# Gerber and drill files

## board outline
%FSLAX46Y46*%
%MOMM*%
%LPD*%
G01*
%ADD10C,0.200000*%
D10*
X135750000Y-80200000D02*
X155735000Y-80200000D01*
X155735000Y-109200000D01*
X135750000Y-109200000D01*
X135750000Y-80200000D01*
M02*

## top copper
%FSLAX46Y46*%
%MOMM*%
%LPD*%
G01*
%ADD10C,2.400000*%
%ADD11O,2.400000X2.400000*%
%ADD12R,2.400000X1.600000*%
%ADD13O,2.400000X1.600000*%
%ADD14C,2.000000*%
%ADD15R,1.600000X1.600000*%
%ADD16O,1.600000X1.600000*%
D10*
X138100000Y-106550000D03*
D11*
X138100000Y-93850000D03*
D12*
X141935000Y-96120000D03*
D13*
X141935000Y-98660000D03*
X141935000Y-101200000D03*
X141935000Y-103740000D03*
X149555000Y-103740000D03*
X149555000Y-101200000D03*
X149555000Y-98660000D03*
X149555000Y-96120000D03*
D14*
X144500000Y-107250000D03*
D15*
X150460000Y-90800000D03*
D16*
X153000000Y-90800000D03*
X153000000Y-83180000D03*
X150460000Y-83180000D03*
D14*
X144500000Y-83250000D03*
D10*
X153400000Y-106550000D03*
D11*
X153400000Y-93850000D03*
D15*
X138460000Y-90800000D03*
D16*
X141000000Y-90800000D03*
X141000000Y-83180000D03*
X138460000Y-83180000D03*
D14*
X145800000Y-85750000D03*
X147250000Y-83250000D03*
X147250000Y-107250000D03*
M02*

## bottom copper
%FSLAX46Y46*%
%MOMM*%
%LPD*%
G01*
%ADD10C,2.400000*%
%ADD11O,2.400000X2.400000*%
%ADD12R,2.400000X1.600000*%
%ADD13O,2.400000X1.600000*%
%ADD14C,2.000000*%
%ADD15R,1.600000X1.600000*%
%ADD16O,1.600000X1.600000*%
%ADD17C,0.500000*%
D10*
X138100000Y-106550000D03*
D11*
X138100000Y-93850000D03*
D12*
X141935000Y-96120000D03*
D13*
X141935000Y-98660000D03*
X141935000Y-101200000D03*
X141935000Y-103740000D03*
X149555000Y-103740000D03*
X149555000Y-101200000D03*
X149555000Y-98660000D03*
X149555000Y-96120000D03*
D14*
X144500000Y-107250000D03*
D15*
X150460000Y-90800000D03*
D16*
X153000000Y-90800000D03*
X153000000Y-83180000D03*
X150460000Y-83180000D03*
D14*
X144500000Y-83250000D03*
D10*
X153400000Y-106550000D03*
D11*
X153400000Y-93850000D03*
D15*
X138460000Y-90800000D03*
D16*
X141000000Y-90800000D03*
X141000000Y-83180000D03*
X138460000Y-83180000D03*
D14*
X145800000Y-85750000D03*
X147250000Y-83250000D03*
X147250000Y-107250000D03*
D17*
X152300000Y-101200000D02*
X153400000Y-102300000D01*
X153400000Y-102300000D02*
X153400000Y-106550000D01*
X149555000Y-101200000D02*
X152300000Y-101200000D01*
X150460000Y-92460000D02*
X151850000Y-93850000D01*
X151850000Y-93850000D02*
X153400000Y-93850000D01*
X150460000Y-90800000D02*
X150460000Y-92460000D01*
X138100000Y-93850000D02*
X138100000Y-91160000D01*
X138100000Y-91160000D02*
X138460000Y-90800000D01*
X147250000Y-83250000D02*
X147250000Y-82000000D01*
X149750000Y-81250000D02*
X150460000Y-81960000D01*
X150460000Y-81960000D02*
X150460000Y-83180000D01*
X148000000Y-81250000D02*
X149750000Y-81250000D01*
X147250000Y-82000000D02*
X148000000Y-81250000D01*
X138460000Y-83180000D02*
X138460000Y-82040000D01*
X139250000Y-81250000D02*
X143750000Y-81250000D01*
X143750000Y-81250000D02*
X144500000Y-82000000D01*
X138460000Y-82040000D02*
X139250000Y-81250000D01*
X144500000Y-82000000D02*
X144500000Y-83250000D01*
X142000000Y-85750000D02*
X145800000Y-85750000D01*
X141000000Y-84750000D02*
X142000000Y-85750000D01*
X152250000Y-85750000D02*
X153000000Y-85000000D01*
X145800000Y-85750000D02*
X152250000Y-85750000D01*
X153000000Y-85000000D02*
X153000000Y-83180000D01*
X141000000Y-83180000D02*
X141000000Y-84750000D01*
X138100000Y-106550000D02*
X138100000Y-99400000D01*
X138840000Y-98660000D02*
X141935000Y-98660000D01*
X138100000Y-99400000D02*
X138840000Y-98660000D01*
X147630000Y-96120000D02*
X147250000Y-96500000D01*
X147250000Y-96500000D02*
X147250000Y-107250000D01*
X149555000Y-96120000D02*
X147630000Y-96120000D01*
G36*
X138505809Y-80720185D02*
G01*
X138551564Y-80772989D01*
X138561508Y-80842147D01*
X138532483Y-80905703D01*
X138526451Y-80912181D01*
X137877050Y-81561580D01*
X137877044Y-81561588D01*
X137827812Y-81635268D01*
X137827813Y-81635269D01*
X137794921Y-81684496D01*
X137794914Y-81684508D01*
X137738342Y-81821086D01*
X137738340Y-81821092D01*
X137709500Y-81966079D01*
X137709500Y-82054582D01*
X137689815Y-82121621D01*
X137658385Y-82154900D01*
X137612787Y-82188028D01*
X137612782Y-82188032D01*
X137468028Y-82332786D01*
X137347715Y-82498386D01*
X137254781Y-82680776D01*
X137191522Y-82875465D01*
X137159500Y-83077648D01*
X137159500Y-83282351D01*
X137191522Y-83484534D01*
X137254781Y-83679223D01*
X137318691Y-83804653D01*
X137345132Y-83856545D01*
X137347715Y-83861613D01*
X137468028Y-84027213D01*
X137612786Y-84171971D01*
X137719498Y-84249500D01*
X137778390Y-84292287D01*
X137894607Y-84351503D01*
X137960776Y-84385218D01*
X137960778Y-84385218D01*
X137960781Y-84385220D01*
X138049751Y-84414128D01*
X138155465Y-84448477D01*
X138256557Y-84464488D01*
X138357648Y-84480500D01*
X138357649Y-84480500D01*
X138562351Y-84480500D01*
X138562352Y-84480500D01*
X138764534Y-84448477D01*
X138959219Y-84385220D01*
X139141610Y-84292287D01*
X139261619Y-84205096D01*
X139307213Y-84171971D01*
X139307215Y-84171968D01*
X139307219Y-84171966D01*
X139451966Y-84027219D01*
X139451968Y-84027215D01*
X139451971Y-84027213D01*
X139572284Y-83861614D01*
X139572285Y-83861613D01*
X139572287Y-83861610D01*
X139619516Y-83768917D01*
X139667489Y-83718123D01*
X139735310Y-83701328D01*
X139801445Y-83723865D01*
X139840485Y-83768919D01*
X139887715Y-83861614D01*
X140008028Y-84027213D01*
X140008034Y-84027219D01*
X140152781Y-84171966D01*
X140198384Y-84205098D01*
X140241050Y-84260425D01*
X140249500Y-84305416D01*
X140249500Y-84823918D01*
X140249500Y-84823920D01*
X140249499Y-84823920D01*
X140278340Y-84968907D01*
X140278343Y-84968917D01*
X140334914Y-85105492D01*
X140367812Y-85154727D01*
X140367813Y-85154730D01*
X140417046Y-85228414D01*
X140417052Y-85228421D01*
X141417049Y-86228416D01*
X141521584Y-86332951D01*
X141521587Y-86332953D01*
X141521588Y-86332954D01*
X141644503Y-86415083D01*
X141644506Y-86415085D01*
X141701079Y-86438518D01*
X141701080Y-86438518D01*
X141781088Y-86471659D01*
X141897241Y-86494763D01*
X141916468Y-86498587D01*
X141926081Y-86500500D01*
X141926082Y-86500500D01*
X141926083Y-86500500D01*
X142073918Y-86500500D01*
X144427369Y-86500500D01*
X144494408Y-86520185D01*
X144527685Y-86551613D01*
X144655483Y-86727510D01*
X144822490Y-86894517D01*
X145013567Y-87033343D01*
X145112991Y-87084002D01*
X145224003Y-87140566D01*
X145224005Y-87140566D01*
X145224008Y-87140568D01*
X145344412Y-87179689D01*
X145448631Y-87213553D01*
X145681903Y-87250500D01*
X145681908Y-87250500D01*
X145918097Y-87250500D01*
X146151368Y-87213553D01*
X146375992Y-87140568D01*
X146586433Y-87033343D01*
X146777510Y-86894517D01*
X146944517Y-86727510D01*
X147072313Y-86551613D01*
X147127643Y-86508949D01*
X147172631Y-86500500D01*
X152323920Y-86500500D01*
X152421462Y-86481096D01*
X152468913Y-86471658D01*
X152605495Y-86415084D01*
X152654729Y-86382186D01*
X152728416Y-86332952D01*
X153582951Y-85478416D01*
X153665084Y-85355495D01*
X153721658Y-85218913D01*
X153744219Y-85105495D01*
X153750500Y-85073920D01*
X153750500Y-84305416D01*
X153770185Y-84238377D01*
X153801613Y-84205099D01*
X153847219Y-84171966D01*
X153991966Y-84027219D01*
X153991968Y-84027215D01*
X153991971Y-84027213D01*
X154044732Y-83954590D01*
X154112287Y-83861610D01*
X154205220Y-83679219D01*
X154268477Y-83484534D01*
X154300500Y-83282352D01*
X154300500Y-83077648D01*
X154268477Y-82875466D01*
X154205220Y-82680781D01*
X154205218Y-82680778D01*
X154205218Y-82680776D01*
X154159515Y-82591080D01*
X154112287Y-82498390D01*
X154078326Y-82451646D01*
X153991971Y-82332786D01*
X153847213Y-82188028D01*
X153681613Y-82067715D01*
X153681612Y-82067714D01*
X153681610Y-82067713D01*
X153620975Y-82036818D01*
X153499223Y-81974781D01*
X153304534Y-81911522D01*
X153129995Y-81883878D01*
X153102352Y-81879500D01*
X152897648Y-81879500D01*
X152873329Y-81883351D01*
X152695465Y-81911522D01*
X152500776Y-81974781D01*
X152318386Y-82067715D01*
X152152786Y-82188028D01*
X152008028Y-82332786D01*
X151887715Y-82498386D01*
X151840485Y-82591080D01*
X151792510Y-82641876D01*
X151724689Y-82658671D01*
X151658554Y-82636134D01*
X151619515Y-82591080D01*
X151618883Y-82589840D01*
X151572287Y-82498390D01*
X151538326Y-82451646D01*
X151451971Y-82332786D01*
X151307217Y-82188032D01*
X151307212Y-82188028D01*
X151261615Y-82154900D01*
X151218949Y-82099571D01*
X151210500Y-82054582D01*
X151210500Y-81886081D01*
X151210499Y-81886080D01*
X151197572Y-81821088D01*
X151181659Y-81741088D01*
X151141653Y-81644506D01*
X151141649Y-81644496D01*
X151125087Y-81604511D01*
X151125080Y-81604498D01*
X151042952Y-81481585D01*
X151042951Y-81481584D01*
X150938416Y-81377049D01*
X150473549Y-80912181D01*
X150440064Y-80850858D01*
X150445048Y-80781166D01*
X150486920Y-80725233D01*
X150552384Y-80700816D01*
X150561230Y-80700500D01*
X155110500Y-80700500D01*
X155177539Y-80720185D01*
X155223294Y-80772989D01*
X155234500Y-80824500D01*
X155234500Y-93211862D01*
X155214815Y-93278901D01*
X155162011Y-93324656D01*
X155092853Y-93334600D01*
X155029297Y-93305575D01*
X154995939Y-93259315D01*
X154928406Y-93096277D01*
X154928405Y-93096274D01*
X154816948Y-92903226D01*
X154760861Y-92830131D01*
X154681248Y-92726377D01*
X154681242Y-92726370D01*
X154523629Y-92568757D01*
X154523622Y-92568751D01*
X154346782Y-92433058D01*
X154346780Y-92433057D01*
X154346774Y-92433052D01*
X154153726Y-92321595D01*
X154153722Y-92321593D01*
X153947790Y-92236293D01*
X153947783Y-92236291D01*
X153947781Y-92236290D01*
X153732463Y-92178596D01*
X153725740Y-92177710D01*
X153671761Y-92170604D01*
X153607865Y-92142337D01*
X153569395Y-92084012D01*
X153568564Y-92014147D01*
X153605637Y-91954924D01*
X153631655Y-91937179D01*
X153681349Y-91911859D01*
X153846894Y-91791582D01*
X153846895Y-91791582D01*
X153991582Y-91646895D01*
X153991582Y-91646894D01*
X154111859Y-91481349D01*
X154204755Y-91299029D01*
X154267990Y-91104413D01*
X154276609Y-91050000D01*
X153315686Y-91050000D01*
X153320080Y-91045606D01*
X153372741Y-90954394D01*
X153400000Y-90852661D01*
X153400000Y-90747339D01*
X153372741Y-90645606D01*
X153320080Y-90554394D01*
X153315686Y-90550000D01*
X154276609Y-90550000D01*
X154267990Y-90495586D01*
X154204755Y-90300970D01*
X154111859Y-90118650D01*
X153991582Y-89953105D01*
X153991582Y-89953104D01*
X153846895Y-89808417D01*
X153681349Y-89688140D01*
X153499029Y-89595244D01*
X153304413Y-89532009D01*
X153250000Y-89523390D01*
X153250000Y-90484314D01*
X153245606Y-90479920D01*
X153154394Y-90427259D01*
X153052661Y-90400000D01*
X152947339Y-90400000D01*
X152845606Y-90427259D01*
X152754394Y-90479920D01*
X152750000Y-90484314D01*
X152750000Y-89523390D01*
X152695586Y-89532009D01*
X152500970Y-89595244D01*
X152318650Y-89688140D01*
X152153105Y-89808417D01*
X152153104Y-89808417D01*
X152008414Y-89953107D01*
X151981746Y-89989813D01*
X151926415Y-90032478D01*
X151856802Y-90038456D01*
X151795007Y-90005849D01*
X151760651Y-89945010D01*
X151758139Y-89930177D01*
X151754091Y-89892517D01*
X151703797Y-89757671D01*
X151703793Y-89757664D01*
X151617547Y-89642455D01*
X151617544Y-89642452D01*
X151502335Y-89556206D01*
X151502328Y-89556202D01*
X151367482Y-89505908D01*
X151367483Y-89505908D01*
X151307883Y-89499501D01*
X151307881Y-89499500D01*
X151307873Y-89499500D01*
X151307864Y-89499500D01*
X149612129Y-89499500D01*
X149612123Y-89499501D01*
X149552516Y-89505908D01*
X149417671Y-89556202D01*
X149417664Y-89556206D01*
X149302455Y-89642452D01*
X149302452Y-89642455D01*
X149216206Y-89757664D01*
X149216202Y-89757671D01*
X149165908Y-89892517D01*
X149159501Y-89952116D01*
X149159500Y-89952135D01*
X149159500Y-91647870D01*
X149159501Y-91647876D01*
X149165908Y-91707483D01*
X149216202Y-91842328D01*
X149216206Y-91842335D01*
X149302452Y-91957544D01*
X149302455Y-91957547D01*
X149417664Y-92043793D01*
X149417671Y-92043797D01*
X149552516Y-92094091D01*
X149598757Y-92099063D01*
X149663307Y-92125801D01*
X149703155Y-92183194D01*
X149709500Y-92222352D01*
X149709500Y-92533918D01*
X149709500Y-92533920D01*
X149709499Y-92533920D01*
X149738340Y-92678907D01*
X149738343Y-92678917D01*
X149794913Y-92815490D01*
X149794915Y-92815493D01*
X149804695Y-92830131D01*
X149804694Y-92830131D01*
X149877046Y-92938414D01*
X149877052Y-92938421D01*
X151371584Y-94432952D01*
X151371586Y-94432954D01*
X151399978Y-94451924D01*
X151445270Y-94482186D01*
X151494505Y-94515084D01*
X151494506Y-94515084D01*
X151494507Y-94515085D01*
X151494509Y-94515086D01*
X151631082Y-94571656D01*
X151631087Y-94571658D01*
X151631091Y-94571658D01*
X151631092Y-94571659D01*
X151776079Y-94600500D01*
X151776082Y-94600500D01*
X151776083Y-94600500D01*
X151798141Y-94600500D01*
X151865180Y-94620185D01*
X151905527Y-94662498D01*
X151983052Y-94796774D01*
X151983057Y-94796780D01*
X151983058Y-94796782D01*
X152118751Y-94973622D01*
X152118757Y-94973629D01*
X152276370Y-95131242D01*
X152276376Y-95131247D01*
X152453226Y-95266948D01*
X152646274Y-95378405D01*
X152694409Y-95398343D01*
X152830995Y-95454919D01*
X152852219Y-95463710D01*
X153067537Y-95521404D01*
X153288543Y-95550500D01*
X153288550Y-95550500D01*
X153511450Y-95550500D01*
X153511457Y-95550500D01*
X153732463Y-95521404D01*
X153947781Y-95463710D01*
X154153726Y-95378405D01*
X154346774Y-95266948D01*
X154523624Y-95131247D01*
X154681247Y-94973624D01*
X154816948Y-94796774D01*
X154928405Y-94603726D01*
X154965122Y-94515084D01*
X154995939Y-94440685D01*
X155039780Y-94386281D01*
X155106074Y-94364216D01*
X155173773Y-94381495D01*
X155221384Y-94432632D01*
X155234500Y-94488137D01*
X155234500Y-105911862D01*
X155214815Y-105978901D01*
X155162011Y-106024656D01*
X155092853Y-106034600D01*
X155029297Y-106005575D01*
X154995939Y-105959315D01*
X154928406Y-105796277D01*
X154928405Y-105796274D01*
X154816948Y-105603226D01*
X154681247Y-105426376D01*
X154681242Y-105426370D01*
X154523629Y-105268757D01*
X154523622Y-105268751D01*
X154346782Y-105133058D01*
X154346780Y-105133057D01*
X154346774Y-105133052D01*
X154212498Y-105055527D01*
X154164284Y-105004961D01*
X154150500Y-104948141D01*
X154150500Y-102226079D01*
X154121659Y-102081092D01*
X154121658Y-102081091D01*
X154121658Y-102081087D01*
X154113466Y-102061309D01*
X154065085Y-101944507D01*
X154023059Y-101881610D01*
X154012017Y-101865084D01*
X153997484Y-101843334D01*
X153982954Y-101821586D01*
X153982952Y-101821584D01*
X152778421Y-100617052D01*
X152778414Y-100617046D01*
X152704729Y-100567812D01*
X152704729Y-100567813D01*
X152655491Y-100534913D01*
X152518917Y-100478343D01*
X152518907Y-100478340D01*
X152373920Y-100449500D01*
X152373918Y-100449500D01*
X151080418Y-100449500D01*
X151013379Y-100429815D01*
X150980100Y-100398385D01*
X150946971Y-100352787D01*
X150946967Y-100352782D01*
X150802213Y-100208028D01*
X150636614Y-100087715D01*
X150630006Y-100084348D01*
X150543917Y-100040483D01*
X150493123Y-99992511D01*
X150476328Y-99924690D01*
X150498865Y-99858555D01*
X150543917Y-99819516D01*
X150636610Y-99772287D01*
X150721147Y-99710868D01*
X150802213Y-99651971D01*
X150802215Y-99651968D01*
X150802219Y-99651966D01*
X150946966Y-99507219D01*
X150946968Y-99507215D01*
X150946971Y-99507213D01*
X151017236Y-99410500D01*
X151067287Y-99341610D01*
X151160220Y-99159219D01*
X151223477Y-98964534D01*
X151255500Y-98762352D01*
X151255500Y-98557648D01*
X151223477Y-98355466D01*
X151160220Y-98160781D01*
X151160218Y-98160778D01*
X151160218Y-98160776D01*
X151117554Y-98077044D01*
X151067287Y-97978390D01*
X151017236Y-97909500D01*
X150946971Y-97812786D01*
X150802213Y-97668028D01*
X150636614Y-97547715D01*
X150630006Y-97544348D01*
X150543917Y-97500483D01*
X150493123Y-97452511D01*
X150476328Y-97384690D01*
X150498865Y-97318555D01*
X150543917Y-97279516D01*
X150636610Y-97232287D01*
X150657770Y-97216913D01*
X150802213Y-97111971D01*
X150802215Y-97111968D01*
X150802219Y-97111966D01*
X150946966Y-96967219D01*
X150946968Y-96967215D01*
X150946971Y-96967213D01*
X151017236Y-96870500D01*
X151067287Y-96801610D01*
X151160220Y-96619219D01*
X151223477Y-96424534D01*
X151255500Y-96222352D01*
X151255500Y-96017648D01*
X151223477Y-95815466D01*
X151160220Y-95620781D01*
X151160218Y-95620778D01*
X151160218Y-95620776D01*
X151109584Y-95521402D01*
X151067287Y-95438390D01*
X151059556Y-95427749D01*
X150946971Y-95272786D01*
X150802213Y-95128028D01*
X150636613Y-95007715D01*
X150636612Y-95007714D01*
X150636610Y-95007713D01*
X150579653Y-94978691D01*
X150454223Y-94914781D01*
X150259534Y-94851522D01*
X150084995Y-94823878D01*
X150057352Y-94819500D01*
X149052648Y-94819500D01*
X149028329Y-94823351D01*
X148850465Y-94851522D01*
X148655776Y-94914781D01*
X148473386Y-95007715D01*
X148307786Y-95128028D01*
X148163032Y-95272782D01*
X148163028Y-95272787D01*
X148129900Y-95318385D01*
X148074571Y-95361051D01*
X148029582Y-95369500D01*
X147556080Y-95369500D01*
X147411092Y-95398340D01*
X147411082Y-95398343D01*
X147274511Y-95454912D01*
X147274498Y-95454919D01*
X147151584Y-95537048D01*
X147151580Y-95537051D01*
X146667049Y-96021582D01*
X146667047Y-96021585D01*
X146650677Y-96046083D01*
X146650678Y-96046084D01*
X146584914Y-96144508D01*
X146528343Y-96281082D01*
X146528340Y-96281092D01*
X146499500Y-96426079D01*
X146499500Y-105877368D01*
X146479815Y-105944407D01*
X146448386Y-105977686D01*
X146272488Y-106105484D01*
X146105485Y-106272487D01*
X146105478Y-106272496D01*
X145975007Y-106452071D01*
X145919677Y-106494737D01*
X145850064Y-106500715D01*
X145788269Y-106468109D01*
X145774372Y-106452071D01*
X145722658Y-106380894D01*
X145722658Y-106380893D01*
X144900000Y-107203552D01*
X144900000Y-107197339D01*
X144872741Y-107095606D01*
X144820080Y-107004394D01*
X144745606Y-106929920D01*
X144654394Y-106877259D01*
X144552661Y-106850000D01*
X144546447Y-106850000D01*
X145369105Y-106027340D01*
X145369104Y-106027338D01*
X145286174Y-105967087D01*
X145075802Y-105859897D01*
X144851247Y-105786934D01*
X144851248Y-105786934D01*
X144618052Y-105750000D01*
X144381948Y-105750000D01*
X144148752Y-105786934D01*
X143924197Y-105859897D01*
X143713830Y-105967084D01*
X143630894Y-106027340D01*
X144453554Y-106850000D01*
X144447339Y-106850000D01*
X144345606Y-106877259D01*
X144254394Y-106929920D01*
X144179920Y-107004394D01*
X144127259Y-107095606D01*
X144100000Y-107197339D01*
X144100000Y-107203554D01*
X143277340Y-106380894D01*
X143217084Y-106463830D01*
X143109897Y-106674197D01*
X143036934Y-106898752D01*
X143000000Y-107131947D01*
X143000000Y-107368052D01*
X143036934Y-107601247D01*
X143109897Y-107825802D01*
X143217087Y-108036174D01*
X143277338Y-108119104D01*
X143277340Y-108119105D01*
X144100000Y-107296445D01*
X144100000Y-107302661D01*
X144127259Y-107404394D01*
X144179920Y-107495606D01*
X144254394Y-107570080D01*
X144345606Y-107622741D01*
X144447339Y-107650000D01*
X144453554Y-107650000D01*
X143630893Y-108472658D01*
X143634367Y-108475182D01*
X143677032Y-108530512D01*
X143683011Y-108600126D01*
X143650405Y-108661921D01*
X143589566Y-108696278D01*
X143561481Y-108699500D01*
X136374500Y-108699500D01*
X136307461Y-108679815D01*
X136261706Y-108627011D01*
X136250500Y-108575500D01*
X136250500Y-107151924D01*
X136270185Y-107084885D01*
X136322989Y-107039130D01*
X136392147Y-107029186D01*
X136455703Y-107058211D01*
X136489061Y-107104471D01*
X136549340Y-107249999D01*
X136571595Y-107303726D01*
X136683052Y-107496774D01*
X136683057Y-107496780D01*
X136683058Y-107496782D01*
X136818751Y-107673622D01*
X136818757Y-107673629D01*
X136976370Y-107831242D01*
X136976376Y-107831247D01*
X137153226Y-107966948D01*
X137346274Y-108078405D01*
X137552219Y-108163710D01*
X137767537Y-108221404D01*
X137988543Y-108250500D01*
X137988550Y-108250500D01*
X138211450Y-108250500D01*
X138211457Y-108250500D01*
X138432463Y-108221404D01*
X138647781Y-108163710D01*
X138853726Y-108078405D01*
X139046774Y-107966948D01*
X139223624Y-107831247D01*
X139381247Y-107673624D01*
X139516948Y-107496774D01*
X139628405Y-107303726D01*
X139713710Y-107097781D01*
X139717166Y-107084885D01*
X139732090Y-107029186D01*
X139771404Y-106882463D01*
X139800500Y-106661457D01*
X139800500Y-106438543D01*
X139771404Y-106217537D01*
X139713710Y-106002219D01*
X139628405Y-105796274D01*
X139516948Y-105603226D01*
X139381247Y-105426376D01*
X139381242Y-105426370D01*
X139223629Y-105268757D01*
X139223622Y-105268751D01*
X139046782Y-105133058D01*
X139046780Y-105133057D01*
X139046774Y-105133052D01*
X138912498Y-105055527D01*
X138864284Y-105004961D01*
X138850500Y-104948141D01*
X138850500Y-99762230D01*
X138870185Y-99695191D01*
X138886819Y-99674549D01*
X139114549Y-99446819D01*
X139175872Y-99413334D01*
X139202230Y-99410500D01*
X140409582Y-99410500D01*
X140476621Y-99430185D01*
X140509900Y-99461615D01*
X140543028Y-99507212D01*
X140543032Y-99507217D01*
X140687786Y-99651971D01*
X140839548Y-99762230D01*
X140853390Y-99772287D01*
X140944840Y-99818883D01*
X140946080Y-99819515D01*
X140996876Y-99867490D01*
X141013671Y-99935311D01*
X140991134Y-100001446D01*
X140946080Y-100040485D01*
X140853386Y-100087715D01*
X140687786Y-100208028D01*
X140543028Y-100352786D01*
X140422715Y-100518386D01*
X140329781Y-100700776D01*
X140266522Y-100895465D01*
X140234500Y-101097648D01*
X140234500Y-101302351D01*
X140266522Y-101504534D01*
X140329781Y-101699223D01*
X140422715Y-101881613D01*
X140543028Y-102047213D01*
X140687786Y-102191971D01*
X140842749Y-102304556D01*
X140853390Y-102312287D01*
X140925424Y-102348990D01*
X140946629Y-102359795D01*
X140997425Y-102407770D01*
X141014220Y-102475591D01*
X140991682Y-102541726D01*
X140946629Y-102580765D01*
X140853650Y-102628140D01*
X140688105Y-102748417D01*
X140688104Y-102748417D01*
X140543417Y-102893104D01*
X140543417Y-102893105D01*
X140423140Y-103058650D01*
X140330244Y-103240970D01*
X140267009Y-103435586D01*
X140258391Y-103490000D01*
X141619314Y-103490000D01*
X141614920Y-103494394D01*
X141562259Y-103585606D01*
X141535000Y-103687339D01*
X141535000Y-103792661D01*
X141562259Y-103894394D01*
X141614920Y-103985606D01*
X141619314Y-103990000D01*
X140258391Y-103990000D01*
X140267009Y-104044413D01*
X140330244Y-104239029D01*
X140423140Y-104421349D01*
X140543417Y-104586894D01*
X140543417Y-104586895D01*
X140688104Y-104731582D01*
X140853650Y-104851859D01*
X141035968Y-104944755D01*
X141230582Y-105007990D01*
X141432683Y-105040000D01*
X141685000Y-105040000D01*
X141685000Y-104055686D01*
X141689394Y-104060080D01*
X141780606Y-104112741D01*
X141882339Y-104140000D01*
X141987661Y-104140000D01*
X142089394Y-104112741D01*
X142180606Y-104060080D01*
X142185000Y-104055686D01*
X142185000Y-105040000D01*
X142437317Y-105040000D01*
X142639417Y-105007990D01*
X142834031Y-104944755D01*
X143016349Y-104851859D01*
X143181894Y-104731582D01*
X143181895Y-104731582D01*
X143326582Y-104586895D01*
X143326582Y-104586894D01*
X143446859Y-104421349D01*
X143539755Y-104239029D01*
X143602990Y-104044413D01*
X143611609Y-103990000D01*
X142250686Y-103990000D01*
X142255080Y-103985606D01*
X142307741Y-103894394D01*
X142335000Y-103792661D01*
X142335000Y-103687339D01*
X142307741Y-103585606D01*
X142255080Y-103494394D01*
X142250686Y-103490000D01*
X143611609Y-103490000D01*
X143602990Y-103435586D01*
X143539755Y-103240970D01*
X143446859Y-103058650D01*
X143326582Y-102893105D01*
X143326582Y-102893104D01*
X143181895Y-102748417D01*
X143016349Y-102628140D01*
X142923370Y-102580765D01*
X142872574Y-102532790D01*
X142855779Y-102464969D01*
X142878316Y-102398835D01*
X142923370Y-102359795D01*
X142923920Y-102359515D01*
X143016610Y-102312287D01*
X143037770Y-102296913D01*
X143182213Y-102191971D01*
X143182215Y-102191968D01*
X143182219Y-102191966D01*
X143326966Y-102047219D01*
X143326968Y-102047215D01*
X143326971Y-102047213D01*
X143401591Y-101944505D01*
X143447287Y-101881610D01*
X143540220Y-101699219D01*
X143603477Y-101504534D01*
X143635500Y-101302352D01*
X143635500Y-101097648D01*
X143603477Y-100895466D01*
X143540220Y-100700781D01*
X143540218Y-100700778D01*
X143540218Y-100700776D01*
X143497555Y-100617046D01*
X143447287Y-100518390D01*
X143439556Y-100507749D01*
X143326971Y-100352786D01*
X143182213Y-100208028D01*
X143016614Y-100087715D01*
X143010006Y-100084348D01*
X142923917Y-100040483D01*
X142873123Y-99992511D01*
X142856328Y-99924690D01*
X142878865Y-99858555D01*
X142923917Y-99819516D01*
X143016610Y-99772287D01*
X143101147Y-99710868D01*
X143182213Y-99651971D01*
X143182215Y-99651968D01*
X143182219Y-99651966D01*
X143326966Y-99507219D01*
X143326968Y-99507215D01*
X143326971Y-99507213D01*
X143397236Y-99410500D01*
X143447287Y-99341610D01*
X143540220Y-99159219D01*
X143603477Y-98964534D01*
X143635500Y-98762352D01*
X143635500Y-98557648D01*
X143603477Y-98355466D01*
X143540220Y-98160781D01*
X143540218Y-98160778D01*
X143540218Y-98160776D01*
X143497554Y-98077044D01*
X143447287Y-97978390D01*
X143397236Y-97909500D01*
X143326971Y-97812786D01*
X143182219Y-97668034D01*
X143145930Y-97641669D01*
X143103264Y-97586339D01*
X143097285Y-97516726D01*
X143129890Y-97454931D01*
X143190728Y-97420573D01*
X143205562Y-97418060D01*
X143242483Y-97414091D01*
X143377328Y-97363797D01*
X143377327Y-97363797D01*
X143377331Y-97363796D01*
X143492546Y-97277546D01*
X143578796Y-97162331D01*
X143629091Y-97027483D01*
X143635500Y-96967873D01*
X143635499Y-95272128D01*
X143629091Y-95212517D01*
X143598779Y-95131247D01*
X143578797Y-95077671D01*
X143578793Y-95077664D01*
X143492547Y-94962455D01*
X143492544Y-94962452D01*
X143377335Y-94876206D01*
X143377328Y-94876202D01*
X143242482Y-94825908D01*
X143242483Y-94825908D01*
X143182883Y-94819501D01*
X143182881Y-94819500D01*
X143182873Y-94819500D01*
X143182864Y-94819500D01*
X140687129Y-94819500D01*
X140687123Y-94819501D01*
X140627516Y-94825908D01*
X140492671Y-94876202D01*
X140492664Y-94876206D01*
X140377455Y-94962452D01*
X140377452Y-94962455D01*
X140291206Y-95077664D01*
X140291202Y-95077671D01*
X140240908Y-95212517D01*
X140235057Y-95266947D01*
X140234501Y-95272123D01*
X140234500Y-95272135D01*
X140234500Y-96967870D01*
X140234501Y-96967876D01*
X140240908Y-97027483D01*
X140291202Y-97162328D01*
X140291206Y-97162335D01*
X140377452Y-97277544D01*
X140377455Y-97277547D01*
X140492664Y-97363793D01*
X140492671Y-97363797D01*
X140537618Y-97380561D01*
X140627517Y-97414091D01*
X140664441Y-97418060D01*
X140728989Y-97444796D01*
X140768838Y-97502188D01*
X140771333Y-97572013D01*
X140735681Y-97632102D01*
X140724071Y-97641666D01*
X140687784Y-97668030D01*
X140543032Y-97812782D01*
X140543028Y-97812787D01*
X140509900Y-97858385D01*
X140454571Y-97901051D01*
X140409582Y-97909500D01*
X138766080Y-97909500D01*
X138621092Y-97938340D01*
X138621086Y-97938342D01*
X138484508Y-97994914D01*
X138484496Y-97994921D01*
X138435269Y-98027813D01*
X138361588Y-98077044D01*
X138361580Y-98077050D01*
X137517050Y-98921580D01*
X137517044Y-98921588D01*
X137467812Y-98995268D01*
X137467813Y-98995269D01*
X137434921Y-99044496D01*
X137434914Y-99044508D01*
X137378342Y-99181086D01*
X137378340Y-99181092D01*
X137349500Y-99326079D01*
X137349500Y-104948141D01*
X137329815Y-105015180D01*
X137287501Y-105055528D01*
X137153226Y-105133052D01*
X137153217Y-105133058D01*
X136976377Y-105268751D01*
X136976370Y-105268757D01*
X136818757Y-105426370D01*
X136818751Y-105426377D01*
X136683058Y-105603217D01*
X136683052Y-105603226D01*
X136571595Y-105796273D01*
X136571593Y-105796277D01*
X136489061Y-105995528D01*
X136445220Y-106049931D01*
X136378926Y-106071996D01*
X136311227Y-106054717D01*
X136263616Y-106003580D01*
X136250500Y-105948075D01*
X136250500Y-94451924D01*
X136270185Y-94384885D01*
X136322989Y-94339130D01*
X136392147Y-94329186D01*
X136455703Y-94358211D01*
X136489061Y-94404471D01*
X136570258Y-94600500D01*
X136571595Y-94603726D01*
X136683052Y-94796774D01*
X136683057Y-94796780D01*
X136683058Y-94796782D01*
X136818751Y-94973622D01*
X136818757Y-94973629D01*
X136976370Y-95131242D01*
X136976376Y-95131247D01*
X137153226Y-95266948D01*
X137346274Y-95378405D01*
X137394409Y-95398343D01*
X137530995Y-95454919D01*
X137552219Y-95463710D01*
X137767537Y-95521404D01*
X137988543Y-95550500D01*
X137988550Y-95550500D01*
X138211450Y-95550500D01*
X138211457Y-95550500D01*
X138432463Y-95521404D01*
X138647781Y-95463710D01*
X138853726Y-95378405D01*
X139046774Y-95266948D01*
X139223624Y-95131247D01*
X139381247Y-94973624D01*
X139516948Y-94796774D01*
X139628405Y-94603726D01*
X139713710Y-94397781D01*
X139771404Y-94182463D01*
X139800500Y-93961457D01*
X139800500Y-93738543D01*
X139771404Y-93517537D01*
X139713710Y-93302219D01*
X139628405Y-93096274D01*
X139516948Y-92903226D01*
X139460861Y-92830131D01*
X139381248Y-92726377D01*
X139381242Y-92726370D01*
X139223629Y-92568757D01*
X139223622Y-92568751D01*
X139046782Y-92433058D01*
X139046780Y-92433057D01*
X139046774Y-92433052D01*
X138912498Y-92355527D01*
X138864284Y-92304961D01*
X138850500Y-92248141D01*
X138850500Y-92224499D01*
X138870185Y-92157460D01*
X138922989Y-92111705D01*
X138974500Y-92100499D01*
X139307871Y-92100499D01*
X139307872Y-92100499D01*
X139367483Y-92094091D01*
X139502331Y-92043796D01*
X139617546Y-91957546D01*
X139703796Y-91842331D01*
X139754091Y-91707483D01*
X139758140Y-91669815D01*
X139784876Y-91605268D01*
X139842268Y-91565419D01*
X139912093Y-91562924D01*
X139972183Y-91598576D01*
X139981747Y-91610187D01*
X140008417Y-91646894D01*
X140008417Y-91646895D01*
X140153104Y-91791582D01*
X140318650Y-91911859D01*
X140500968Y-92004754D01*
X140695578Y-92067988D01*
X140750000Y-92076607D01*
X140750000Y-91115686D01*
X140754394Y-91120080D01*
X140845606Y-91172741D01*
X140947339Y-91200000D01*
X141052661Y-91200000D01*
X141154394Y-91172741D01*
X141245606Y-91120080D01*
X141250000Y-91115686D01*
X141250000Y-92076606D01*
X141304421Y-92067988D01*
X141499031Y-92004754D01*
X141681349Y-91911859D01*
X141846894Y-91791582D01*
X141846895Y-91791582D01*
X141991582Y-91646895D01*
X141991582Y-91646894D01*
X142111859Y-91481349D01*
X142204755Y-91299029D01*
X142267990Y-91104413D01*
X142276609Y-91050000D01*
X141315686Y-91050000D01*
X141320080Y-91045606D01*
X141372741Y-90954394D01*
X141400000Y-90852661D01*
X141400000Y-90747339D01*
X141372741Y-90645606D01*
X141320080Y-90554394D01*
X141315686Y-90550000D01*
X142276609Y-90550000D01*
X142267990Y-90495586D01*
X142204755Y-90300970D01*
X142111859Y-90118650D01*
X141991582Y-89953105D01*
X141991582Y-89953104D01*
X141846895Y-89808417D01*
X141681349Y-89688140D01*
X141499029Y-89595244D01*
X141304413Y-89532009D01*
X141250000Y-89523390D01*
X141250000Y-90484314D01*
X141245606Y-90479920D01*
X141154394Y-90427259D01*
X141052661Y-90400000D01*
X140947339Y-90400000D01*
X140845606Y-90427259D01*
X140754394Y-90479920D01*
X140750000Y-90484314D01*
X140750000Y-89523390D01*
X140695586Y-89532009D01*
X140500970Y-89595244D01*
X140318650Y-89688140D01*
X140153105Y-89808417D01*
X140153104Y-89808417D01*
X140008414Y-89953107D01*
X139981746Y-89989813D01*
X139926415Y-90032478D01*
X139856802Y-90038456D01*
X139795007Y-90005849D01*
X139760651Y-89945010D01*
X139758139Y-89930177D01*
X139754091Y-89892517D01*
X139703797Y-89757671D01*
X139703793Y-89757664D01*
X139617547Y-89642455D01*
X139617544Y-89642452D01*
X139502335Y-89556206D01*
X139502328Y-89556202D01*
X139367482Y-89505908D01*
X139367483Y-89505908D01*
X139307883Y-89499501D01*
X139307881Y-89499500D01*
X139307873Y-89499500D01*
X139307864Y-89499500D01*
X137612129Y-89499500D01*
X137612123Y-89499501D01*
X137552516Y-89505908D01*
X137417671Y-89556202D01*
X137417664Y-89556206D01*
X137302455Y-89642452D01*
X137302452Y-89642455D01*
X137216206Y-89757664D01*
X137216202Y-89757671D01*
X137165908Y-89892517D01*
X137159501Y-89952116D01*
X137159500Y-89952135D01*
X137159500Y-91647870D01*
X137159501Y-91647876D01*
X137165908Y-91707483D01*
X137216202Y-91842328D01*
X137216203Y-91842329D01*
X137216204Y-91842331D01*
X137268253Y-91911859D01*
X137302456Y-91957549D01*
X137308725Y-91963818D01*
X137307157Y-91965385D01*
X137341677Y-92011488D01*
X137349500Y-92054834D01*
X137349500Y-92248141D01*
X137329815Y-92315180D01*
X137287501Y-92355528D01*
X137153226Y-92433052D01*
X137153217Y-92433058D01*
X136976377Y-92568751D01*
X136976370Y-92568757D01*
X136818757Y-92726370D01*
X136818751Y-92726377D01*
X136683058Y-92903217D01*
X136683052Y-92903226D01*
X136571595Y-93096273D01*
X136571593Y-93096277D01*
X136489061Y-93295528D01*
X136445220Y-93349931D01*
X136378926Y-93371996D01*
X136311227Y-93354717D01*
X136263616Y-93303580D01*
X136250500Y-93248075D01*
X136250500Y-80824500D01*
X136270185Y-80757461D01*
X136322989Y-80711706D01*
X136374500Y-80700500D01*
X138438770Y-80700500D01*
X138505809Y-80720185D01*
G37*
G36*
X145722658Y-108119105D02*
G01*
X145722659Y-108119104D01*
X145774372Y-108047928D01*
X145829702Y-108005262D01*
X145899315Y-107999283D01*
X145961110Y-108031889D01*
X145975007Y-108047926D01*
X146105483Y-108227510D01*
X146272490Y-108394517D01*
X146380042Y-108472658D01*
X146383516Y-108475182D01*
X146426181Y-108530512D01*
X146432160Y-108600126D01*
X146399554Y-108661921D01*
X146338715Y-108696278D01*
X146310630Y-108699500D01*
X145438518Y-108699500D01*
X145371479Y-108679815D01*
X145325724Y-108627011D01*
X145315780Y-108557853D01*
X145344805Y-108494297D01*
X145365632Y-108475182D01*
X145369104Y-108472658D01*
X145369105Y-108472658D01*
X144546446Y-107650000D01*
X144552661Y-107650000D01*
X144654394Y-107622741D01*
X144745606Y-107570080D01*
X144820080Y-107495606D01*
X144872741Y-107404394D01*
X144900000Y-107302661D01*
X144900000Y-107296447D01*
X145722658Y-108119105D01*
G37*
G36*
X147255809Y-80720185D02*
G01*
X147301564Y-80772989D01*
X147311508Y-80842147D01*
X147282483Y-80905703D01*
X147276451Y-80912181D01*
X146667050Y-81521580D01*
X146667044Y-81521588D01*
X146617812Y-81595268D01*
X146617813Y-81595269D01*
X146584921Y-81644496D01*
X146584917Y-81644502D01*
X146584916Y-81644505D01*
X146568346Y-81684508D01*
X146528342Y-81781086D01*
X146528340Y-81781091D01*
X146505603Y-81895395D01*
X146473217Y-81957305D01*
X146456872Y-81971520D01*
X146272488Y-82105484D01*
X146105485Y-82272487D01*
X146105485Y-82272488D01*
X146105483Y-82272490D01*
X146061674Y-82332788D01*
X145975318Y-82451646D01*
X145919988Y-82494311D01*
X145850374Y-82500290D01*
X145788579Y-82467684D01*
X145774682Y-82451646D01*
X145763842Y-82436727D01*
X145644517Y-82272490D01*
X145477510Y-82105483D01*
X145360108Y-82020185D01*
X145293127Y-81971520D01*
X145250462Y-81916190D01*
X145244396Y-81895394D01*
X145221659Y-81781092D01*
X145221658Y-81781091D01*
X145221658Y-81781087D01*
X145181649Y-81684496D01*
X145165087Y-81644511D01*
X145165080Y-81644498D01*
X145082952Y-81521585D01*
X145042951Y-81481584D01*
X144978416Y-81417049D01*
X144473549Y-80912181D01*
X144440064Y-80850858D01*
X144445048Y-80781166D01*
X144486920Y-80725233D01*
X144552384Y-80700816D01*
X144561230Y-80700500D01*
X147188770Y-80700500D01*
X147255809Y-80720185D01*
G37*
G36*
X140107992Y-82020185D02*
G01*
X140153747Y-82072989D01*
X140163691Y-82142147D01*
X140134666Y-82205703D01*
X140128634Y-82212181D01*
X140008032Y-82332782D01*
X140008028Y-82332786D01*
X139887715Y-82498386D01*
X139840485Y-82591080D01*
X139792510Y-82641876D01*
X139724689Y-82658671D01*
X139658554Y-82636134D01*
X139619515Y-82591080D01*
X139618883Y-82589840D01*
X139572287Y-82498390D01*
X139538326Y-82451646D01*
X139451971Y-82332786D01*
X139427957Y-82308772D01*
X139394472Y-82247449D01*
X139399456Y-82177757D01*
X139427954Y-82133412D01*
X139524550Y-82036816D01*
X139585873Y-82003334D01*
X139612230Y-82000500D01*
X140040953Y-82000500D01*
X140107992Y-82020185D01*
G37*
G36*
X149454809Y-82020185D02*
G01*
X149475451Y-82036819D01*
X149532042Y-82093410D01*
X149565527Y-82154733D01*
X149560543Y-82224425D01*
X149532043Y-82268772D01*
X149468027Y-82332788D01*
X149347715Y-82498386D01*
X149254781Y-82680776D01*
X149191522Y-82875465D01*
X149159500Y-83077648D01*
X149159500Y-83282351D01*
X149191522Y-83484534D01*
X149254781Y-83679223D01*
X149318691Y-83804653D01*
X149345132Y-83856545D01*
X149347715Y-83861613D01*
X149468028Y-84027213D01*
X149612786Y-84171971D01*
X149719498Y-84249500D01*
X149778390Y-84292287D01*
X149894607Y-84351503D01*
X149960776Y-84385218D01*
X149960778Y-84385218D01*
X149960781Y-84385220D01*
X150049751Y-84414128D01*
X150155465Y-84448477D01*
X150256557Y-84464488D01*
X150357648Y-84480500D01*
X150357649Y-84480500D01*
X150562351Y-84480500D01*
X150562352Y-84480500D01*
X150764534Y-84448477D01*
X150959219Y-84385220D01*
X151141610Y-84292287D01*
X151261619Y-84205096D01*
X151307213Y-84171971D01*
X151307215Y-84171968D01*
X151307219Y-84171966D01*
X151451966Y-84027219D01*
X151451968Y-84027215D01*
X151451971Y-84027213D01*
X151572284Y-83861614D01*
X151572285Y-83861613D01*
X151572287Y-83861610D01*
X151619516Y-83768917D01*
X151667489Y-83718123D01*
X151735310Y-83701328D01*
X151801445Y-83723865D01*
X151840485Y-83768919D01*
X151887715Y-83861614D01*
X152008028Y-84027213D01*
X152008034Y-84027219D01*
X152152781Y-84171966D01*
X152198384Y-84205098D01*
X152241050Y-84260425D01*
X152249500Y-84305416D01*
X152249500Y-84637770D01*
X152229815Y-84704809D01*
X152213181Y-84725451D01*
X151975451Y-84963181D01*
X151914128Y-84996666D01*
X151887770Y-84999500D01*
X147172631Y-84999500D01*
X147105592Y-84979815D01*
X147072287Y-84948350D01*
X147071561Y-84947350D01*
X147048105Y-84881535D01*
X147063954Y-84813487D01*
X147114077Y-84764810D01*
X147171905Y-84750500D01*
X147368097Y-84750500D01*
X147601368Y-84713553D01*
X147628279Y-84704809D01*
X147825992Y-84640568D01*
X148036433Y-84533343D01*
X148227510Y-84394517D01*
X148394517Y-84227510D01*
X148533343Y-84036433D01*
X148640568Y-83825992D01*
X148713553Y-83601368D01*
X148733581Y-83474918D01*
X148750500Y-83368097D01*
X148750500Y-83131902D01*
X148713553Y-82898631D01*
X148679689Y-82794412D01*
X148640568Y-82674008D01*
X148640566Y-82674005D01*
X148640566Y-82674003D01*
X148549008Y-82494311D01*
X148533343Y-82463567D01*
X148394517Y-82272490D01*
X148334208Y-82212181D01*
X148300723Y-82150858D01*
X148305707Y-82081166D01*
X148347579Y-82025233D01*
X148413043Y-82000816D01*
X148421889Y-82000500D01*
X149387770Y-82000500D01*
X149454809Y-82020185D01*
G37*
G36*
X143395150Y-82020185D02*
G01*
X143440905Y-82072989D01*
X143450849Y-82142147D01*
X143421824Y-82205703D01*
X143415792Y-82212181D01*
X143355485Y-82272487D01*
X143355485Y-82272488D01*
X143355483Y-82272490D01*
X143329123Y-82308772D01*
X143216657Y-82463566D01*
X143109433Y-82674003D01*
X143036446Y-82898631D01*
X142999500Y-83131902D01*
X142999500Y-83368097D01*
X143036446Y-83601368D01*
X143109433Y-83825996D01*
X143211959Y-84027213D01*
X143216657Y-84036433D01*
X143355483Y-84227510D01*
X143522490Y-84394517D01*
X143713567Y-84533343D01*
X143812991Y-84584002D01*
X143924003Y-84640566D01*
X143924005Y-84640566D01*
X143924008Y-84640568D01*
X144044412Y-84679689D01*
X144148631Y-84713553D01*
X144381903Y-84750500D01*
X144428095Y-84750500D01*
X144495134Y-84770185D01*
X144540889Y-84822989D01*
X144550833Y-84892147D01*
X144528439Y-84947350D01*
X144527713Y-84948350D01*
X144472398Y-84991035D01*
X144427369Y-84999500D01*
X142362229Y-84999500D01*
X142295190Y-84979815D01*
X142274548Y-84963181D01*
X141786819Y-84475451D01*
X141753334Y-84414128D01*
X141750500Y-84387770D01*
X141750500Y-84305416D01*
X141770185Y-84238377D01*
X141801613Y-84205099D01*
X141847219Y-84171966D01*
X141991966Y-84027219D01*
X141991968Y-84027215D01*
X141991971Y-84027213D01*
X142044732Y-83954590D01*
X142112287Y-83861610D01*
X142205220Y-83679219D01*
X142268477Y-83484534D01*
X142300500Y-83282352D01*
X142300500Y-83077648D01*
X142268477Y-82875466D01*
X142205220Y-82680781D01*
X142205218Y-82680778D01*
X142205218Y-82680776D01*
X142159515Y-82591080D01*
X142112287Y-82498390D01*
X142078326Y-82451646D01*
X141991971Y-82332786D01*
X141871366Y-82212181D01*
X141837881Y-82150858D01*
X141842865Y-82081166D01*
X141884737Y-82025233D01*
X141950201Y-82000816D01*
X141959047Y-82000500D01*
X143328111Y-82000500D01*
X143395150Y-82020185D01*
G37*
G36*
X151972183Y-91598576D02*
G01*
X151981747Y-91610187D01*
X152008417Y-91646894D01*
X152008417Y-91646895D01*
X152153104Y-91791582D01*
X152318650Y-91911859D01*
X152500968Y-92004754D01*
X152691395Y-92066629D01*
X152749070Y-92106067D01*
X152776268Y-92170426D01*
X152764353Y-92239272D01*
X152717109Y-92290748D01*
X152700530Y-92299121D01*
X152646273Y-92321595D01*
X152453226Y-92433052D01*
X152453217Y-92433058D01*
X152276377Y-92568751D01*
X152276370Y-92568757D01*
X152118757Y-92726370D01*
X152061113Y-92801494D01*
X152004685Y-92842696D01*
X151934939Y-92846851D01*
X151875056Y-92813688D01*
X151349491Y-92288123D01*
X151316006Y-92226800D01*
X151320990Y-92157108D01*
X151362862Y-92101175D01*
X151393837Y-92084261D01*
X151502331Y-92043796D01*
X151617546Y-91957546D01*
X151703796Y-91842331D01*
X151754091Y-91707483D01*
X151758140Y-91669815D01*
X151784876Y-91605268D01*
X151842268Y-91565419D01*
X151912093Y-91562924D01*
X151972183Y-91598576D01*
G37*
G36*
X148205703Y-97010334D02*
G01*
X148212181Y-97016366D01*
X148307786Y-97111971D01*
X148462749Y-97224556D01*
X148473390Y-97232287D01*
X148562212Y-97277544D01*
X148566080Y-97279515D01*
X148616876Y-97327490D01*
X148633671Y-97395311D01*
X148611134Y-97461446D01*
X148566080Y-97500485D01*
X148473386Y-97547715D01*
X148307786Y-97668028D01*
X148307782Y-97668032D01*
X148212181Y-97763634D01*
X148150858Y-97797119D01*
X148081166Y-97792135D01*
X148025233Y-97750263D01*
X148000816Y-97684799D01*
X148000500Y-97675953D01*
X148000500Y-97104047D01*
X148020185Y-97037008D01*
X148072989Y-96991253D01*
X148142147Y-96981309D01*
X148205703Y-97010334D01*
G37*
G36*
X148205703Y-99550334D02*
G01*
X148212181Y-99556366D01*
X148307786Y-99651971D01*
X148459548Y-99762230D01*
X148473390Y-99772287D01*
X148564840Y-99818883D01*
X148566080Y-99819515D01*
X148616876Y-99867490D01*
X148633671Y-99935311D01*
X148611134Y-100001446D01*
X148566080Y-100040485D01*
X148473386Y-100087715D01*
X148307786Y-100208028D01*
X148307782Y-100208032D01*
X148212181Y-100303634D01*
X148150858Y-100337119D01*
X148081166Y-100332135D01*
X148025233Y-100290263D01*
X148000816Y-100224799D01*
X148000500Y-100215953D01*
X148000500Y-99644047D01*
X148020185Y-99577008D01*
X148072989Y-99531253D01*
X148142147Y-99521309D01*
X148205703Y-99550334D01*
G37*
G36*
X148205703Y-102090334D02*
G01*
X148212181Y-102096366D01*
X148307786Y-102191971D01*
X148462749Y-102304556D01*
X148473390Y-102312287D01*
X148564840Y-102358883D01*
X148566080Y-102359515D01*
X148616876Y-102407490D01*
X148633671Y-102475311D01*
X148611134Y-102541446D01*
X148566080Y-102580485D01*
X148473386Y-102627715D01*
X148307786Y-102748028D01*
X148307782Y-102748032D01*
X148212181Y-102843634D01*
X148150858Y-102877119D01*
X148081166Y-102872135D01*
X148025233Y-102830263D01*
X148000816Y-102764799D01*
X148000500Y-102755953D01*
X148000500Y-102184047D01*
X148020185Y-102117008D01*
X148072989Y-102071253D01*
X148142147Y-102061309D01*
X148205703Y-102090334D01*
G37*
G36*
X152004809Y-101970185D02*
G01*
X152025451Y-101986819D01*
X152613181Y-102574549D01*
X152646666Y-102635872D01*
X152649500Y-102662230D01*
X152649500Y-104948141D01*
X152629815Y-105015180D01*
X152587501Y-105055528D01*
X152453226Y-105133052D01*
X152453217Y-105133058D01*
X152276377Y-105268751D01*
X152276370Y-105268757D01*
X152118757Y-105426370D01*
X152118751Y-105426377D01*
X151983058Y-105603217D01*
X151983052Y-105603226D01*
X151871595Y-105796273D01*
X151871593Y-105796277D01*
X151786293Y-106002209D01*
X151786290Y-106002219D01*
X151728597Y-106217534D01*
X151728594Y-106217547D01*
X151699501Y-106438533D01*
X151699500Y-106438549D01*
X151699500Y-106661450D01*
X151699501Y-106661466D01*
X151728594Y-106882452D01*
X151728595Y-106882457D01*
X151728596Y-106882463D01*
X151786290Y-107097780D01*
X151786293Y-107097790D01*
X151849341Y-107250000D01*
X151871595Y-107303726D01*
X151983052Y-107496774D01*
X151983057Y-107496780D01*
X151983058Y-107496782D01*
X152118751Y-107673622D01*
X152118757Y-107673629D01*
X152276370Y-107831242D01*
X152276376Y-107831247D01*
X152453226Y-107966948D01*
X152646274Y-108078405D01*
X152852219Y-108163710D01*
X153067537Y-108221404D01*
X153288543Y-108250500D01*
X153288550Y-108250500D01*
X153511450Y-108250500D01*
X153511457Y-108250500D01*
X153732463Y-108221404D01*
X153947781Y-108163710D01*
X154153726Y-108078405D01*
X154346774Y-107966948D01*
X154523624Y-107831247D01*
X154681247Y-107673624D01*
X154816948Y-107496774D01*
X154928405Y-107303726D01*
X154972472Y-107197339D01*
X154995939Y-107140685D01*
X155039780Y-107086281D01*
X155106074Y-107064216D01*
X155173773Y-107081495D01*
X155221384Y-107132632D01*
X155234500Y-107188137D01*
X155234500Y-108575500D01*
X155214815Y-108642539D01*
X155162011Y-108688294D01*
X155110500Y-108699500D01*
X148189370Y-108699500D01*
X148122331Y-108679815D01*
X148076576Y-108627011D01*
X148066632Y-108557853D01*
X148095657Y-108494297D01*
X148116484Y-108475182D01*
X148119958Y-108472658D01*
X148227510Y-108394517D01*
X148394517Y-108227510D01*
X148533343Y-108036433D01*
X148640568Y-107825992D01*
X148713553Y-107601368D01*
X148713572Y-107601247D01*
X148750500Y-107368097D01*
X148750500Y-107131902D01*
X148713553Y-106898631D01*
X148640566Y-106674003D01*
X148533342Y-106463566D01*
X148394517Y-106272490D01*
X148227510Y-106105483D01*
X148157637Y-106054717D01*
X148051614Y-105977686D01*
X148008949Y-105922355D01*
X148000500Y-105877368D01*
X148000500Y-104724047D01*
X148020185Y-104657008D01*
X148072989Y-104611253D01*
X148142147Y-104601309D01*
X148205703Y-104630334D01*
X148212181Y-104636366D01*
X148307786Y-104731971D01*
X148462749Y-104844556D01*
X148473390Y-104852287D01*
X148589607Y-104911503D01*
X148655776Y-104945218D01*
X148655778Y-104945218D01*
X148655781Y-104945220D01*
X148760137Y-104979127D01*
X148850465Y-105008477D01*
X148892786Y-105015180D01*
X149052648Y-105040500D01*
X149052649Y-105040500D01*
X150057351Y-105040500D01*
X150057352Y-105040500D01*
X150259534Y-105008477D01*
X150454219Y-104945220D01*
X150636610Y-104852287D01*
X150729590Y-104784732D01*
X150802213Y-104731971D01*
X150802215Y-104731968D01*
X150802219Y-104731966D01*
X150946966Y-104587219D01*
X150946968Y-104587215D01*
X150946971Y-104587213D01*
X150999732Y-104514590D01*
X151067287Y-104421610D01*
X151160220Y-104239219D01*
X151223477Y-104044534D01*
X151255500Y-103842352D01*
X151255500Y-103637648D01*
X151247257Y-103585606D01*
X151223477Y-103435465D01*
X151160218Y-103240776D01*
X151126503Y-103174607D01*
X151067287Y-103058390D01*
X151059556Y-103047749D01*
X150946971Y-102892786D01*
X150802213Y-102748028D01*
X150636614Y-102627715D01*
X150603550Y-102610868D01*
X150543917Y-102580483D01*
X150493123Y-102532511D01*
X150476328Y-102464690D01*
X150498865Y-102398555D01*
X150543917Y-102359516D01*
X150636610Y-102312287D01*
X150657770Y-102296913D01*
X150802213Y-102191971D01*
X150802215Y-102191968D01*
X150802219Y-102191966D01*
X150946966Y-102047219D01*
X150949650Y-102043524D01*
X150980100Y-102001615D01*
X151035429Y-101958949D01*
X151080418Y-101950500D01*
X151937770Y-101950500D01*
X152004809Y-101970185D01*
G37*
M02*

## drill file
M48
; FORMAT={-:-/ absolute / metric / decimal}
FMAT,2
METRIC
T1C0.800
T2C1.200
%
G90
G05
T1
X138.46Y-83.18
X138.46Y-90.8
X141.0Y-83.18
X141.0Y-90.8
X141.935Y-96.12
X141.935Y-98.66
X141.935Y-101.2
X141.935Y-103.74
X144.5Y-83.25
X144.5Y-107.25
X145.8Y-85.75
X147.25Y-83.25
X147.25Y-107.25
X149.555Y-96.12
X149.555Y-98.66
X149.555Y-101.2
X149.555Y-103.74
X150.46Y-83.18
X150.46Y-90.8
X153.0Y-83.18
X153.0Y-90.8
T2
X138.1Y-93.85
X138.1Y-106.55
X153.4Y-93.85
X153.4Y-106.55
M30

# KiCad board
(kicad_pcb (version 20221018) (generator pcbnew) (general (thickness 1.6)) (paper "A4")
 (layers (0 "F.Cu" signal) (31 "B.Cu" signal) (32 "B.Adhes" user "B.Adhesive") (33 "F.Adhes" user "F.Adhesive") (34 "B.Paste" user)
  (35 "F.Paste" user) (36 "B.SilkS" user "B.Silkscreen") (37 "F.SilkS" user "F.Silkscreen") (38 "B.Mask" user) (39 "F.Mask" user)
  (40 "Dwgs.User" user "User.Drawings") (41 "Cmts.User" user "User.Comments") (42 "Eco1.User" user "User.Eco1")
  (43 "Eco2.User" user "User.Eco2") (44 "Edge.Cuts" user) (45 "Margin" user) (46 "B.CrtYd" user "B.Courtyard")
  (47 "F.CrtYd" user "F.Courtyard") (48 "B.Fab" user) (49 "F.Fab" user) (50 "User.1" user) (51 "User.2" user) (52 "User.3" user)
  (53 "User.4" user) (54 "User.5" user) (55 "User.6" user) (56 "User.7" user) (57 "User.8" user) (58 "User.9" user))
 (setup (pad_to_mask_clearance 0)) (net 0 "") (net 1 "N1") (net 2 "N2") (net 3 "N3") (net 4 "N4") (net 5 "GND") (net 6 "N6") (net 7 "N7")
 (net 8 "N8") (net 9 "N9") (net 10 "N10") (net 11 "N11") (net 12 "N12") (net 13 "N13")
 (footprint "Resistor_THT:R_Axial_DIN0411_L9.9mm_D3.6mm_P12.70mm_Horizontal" (layer "F.Cu") (at 138.1 106.55 90)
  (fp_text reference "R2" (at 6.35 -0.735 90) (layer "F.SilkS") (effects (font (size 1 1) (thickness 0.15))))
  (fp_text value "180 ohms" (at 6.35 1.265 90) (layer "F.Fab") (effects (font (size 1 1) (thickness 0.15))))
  (pad "1" thru_hole circle (at 0 0 90) (size 2.4 2.4) (drill 1.2) (layers "*.Cu" "*.Mask") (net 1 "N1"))
  (pad "2" thru_hole oval (at 12.7 0 90) (size 2.4 2.4) (drill 1.2) (layers "*.Cu" "*.Mask") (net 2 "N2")))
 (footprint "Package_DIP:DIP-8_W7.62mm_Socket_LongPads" (layer "F.Cu") (at 141.935 96.12)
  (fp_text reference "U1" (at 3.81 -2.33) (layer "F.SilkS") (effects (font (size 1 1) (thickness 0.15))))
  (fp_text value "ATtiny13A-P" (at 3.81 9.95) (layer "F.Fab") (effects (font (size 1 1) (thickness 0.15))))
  (pad "1" thru_hole rect (at 0 0) (size 2.4 1.6) (drill 0.8) (layers "*.Cu" "*.Mask") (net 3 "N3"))
  (pad "2" thru_hole oval (at 0 2.54) (size 2.4 1.6) (drill 0.8) (layers "*.Cu" "*.Mask") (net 1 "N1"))
  (pad "3" thru_hole oval (at 0 5.08) (size 2.4 1.6) (drill 0.8) (layers "*.Cu" "*.Mask") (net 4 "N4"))
  (pad "4" thru_hole oval (at 0 7.62) (size 2.4 1.6) (drill 0.8) (layers "*.Cu" "*.Mask") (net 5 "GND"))
  (pad "5" thru_hole oval (at 7.62 7.62) (size 2.4 1.6) (drill 0.8) (layers "*.Cu" "*.Mask") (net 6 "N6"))
  (pad "6" thru_hole oval (at 7.62 5.08) (size 2.4 1.6) (drill 0.8) (layers "*.Cu" "*.Mask") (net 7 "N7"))
  (pad "7" thru_hole oval (at 7.62 2.54) (size 2.4 1.6) (drill 0.8) (layers "*.Cu" "*.Mask") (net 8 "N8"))
  (pad "8" thru_hole oval (at 7.62 0) (size 2.4 1.6) (drill 0.8) (layers "*.Cu" "*.Mask") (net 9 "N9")))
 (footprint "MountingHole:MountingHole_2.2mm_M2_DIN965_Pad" (layer "F.Cu") (at 144.5 107.25 180)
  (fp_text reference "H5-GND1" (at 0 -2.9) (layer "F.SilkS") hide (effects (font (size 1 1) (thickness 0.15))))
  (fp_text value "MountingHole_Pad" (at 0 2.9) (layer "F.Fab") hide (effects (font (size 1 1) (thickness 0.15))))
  (pad "1" thru_hole circle (at 0 0 180) (size 2 2) (drill 0.8) (layers "*.Cu" "*.Mask") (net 5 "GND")))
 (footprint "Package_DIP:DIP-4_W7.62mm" (layer "F.Cu") (at 150.46 90.8 90)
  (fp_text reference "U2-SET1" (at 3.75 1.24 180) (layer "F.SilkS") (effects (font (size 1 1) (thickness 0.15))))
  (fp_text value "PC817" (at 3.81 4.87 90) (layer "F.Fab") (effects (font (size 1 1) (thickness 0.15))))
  (pad "1" thru_hole rect (at 0 0 90) (size 1.6 1.6) (drill 0.8) (layers "*.Cu" "*.Mask") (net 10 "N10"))
  (pad "2" thru_hole oval (at 0 2.54 90) (size 1.6 1.6) (drill 0.8) (layers "*.Cu" "*.Mask") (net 5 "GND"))
  (pad "3" thru_hole oval (at 7.62 2.54 90) (size 1.6 1.6) (drill 0.8) (layers "*.Cu" "*.Mask") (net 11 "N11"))
  (pad "4" thru_hole oval (at 7.62 0 90) (size 1.6 1.6) (drill 0.8) (layers "*.Cu" "*.Mask") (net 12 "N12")))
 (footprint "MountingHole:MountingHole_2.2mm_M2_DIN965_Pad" (layer "F.Cu") (at 132.5 86.75)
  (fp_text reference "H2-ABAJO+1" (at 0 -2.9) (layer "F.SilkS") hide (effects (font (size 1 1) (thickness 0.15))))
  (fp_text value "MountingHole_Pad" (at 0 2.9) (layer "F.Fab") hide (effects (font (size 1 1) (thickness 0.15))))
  (pad "1" thru_hole circle (at 12 -3.5) (size 2 2) (drill 0.8) (layers "*.Cu" "*.Mask") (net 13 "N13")))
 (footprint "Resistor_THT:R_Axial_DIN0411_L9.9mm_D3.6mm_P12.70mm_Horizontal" (layer "F.Cu") (at 153.4 106.55 90)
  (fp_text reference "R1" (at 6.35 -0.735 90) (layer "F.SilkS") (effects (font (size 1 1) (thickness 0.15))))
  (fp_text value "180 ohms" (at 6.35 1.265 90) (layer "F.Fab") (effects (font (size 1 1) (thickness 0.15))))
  (pad "1" thru_hole circle (at 0 0 90) (size 2.4 2.4) (drill 1.2) (layers "*.Cu" "*.Mask") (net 7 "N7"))
  (pad "2" thru_hole oval (at 12.7 0 90) (size 2.4 2.4) (drill 1.2) (layers "*.Cu" "*.Mask") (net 10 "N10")))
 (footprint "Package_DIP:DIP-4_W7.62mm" (layer "F.Cu") (at 138.46 90.8 90)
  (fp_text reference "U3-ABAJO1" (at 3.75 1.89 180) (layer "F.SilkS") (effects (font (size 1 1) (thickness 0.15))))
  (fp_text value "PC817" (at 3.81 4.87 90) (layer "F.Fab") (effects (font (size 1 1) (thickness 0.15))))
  (pad "1" thru_hole rect (at 0 0 90) (size 1.6 1.6) (drill 0.8) (layers "*.Cu" "*.Mask") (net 2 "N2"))
  (pad "2" thru_hole oval (at 0 2.54 90) (size 1.6 1.6) (drill 0.8) (layers "*.Cu" "*.Mask") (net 5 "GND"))
  (pad "3" thru_hole oval (at 7.62 2.54 90) (size 1.6 1.6) (drill 0.8) (layers "*.Cu" "*.Mask") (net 11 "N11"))
  (pad "4" thru_hole oval (at 7.62 0 90) (size 1.6 1.6) (drill 0.8) (layers "*.Cu" "*.Mask") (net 13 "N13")))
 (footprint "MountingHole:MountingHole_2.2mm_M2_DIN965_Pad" (layer "F.Cu") (at 145.8 85.75)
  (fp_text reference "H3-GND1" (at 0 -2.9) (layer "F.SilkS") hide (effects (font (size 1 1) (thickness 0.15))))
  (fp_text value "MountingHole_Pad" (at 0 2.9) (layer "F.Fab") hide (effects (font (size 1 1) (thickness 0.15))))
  (pad "1" thru_hole circle (at 0 0) (size 2 2) (drill 0.8) (layers "*.Cu" "*.Mask") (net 11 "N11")))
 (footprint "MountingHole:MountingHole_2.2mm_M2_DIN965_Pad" (layer "F.Cu") (at 132.5 81.4)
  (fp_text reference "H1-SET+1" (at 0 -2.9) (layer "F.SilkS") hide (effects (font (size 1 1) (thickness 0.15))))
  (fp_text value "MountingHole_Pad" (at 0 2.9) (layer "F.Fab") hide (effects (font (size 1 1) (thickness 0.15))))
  (pad "1" thru_hole circle (at 14.75 1.85) (size 2 2) (drill 0.8) (layers "*.Cu" "*.Mask") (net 12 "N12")))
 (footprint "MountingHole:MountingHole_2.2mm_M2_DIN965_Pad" (layer "F.Cu") (at 147.25 107.25 180)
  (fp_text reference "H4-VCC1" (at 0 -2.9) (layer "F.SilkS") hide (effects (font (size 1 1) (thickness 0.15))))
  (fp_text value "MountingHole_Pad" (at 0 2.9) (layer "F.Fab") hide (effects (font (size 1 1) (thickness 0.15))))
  (pad "1" thru_hole circle (at 0 0 180) (size 2 2) (drill 0.8) (layers "*.Cu" "*.Mask") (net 9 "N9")))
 (gr_rect (start 135.75 80.2) (end 155.735 109.2) (stroke (width 0.2) (type default)) (fill none) (layer "Edge.Cuts"))
 (segment (start 152.3 101.2) (end 153.4 102.3) (width 0.5) (layer "B.Cu") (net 7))
 (segment (start 153.4 102.3) (end 153.4 106.55) (width 0.5) (layer "B.Cu") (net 7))
 (segment (start 149.555 101.2) (end 152.3 101.2) (width 0.5) (layer "B.Cu") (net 7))
 (segment (start 150.46 92.46) (end 151.85 93.85) (width 0.5) (layer "B.Cu") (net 10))
 (segment (start 151.85 93.85) (end 153.4 93.85) (width 0.5) (layer "B.Cu") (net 10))
 (segment (start 150.46 90.8) (end 150.46 92.46) (width 0.5) (layer "B.Cu") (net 10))
 (segment (start 138.1 93.85) (end 138.1 91.16) (width 0.5) (layer "B.Cu") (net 2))
 (segment (start 138.1 91.16) (end 138.46 90.8) (width 0.5) (layer "B.Cu") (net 2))
 (segment (start 147.25 83.25) (end 147.25 82) (width 0.5) (layer "B.Cu") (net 12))
 (segment (start 149.75 81.25) (end 150.46 81.96) (width 0.5) (layer "B.Cu") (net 12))
 (segment (start 150.46 81.96) (end 150.46 83.18) (width 0.5) (layer "B.Cu") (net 12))
 (segment (start 148 81.25) (end 149.75 81.25) (width 0.5) (layer "B.Cu") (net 12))
 (segment (start 147.25 82) (end 148 81.25) (width 0.5) (layer "B.Cu") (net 12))
 (segment (start 138.46 83.18) (end 138.46 82.04) (width 0.5) (layer "B.Cu") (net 13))
 (segment (start 139.25 81.25) (end 143.75 81.25) (width 0.5) (layer "B.Cu") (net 13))
 (segment (start 143.75 81.25) (end 144.5 82) (width 0.5) (layer "B.Cu") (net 13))
 (segment (start 138.46 82.04) (end 139.25 81.25) (width 0.5) (layer "B.Cu") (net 13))
 (segment (start 144.5 82) (end 144.5 83.25) (width 0.5) (layer "B.Cu") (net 13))
 (segment (start 142 85.75) (end 145.8 85.75) (width 0.5) (layer "B.Cu") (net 11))
 (segment (start 141 84.75) (end 142 85.75) (width 0.5) (layer "B.Cu") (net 11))
 (segment (start 152.25 85.75) (end 153 85) (width 0.5) (layer "B.Cu") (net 11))
 (segment (start 145.8 85.75) (end 152.25 85.75) (width 0.5) (layer "B.Cu") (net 11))
 (segment (start 153 85) (end 153 83.18) (width 0.5) (layer "B.Cu") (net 11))
 (segment (start 141 83.18) (end 141 84.75) (width 0.5) (layer "B.Cu") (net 11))
 (segment (start 138.1 106.55) (end 138.1 99.4) (width 0.5) (layer "B.Cu") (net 1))
 (segment (start 138.84 98.66) (end 141.935 98.66) (width 0.5) (layer "B.Cu") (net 1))
 (segment (start 138.1 99.4) (end 138.84 98.66) (width 0.5) (layer "B.Cu") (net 1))
 (segment (start 147.63 96.12) (end 147.25 96.5) (width 0.5) (layer "B.Cu") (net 9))
 (segment (start 147.25 96.5) (end 147.25 107.25) (width 0.5) (layer "B.Cu") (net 9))
 (segment (start 149.555 96.12) (end 147.63 96.12) (width 0.5) (layer "B.Cu") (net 9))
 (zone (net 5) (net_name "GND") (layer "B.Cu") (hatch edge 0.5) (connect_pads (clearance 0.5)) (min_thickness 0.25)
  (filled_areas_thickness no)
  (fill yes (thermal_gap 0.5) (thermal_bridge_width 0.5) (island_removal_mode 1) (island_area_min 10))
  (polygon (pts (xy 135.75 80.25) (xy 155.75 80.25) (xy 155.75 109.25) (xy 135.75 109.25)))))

